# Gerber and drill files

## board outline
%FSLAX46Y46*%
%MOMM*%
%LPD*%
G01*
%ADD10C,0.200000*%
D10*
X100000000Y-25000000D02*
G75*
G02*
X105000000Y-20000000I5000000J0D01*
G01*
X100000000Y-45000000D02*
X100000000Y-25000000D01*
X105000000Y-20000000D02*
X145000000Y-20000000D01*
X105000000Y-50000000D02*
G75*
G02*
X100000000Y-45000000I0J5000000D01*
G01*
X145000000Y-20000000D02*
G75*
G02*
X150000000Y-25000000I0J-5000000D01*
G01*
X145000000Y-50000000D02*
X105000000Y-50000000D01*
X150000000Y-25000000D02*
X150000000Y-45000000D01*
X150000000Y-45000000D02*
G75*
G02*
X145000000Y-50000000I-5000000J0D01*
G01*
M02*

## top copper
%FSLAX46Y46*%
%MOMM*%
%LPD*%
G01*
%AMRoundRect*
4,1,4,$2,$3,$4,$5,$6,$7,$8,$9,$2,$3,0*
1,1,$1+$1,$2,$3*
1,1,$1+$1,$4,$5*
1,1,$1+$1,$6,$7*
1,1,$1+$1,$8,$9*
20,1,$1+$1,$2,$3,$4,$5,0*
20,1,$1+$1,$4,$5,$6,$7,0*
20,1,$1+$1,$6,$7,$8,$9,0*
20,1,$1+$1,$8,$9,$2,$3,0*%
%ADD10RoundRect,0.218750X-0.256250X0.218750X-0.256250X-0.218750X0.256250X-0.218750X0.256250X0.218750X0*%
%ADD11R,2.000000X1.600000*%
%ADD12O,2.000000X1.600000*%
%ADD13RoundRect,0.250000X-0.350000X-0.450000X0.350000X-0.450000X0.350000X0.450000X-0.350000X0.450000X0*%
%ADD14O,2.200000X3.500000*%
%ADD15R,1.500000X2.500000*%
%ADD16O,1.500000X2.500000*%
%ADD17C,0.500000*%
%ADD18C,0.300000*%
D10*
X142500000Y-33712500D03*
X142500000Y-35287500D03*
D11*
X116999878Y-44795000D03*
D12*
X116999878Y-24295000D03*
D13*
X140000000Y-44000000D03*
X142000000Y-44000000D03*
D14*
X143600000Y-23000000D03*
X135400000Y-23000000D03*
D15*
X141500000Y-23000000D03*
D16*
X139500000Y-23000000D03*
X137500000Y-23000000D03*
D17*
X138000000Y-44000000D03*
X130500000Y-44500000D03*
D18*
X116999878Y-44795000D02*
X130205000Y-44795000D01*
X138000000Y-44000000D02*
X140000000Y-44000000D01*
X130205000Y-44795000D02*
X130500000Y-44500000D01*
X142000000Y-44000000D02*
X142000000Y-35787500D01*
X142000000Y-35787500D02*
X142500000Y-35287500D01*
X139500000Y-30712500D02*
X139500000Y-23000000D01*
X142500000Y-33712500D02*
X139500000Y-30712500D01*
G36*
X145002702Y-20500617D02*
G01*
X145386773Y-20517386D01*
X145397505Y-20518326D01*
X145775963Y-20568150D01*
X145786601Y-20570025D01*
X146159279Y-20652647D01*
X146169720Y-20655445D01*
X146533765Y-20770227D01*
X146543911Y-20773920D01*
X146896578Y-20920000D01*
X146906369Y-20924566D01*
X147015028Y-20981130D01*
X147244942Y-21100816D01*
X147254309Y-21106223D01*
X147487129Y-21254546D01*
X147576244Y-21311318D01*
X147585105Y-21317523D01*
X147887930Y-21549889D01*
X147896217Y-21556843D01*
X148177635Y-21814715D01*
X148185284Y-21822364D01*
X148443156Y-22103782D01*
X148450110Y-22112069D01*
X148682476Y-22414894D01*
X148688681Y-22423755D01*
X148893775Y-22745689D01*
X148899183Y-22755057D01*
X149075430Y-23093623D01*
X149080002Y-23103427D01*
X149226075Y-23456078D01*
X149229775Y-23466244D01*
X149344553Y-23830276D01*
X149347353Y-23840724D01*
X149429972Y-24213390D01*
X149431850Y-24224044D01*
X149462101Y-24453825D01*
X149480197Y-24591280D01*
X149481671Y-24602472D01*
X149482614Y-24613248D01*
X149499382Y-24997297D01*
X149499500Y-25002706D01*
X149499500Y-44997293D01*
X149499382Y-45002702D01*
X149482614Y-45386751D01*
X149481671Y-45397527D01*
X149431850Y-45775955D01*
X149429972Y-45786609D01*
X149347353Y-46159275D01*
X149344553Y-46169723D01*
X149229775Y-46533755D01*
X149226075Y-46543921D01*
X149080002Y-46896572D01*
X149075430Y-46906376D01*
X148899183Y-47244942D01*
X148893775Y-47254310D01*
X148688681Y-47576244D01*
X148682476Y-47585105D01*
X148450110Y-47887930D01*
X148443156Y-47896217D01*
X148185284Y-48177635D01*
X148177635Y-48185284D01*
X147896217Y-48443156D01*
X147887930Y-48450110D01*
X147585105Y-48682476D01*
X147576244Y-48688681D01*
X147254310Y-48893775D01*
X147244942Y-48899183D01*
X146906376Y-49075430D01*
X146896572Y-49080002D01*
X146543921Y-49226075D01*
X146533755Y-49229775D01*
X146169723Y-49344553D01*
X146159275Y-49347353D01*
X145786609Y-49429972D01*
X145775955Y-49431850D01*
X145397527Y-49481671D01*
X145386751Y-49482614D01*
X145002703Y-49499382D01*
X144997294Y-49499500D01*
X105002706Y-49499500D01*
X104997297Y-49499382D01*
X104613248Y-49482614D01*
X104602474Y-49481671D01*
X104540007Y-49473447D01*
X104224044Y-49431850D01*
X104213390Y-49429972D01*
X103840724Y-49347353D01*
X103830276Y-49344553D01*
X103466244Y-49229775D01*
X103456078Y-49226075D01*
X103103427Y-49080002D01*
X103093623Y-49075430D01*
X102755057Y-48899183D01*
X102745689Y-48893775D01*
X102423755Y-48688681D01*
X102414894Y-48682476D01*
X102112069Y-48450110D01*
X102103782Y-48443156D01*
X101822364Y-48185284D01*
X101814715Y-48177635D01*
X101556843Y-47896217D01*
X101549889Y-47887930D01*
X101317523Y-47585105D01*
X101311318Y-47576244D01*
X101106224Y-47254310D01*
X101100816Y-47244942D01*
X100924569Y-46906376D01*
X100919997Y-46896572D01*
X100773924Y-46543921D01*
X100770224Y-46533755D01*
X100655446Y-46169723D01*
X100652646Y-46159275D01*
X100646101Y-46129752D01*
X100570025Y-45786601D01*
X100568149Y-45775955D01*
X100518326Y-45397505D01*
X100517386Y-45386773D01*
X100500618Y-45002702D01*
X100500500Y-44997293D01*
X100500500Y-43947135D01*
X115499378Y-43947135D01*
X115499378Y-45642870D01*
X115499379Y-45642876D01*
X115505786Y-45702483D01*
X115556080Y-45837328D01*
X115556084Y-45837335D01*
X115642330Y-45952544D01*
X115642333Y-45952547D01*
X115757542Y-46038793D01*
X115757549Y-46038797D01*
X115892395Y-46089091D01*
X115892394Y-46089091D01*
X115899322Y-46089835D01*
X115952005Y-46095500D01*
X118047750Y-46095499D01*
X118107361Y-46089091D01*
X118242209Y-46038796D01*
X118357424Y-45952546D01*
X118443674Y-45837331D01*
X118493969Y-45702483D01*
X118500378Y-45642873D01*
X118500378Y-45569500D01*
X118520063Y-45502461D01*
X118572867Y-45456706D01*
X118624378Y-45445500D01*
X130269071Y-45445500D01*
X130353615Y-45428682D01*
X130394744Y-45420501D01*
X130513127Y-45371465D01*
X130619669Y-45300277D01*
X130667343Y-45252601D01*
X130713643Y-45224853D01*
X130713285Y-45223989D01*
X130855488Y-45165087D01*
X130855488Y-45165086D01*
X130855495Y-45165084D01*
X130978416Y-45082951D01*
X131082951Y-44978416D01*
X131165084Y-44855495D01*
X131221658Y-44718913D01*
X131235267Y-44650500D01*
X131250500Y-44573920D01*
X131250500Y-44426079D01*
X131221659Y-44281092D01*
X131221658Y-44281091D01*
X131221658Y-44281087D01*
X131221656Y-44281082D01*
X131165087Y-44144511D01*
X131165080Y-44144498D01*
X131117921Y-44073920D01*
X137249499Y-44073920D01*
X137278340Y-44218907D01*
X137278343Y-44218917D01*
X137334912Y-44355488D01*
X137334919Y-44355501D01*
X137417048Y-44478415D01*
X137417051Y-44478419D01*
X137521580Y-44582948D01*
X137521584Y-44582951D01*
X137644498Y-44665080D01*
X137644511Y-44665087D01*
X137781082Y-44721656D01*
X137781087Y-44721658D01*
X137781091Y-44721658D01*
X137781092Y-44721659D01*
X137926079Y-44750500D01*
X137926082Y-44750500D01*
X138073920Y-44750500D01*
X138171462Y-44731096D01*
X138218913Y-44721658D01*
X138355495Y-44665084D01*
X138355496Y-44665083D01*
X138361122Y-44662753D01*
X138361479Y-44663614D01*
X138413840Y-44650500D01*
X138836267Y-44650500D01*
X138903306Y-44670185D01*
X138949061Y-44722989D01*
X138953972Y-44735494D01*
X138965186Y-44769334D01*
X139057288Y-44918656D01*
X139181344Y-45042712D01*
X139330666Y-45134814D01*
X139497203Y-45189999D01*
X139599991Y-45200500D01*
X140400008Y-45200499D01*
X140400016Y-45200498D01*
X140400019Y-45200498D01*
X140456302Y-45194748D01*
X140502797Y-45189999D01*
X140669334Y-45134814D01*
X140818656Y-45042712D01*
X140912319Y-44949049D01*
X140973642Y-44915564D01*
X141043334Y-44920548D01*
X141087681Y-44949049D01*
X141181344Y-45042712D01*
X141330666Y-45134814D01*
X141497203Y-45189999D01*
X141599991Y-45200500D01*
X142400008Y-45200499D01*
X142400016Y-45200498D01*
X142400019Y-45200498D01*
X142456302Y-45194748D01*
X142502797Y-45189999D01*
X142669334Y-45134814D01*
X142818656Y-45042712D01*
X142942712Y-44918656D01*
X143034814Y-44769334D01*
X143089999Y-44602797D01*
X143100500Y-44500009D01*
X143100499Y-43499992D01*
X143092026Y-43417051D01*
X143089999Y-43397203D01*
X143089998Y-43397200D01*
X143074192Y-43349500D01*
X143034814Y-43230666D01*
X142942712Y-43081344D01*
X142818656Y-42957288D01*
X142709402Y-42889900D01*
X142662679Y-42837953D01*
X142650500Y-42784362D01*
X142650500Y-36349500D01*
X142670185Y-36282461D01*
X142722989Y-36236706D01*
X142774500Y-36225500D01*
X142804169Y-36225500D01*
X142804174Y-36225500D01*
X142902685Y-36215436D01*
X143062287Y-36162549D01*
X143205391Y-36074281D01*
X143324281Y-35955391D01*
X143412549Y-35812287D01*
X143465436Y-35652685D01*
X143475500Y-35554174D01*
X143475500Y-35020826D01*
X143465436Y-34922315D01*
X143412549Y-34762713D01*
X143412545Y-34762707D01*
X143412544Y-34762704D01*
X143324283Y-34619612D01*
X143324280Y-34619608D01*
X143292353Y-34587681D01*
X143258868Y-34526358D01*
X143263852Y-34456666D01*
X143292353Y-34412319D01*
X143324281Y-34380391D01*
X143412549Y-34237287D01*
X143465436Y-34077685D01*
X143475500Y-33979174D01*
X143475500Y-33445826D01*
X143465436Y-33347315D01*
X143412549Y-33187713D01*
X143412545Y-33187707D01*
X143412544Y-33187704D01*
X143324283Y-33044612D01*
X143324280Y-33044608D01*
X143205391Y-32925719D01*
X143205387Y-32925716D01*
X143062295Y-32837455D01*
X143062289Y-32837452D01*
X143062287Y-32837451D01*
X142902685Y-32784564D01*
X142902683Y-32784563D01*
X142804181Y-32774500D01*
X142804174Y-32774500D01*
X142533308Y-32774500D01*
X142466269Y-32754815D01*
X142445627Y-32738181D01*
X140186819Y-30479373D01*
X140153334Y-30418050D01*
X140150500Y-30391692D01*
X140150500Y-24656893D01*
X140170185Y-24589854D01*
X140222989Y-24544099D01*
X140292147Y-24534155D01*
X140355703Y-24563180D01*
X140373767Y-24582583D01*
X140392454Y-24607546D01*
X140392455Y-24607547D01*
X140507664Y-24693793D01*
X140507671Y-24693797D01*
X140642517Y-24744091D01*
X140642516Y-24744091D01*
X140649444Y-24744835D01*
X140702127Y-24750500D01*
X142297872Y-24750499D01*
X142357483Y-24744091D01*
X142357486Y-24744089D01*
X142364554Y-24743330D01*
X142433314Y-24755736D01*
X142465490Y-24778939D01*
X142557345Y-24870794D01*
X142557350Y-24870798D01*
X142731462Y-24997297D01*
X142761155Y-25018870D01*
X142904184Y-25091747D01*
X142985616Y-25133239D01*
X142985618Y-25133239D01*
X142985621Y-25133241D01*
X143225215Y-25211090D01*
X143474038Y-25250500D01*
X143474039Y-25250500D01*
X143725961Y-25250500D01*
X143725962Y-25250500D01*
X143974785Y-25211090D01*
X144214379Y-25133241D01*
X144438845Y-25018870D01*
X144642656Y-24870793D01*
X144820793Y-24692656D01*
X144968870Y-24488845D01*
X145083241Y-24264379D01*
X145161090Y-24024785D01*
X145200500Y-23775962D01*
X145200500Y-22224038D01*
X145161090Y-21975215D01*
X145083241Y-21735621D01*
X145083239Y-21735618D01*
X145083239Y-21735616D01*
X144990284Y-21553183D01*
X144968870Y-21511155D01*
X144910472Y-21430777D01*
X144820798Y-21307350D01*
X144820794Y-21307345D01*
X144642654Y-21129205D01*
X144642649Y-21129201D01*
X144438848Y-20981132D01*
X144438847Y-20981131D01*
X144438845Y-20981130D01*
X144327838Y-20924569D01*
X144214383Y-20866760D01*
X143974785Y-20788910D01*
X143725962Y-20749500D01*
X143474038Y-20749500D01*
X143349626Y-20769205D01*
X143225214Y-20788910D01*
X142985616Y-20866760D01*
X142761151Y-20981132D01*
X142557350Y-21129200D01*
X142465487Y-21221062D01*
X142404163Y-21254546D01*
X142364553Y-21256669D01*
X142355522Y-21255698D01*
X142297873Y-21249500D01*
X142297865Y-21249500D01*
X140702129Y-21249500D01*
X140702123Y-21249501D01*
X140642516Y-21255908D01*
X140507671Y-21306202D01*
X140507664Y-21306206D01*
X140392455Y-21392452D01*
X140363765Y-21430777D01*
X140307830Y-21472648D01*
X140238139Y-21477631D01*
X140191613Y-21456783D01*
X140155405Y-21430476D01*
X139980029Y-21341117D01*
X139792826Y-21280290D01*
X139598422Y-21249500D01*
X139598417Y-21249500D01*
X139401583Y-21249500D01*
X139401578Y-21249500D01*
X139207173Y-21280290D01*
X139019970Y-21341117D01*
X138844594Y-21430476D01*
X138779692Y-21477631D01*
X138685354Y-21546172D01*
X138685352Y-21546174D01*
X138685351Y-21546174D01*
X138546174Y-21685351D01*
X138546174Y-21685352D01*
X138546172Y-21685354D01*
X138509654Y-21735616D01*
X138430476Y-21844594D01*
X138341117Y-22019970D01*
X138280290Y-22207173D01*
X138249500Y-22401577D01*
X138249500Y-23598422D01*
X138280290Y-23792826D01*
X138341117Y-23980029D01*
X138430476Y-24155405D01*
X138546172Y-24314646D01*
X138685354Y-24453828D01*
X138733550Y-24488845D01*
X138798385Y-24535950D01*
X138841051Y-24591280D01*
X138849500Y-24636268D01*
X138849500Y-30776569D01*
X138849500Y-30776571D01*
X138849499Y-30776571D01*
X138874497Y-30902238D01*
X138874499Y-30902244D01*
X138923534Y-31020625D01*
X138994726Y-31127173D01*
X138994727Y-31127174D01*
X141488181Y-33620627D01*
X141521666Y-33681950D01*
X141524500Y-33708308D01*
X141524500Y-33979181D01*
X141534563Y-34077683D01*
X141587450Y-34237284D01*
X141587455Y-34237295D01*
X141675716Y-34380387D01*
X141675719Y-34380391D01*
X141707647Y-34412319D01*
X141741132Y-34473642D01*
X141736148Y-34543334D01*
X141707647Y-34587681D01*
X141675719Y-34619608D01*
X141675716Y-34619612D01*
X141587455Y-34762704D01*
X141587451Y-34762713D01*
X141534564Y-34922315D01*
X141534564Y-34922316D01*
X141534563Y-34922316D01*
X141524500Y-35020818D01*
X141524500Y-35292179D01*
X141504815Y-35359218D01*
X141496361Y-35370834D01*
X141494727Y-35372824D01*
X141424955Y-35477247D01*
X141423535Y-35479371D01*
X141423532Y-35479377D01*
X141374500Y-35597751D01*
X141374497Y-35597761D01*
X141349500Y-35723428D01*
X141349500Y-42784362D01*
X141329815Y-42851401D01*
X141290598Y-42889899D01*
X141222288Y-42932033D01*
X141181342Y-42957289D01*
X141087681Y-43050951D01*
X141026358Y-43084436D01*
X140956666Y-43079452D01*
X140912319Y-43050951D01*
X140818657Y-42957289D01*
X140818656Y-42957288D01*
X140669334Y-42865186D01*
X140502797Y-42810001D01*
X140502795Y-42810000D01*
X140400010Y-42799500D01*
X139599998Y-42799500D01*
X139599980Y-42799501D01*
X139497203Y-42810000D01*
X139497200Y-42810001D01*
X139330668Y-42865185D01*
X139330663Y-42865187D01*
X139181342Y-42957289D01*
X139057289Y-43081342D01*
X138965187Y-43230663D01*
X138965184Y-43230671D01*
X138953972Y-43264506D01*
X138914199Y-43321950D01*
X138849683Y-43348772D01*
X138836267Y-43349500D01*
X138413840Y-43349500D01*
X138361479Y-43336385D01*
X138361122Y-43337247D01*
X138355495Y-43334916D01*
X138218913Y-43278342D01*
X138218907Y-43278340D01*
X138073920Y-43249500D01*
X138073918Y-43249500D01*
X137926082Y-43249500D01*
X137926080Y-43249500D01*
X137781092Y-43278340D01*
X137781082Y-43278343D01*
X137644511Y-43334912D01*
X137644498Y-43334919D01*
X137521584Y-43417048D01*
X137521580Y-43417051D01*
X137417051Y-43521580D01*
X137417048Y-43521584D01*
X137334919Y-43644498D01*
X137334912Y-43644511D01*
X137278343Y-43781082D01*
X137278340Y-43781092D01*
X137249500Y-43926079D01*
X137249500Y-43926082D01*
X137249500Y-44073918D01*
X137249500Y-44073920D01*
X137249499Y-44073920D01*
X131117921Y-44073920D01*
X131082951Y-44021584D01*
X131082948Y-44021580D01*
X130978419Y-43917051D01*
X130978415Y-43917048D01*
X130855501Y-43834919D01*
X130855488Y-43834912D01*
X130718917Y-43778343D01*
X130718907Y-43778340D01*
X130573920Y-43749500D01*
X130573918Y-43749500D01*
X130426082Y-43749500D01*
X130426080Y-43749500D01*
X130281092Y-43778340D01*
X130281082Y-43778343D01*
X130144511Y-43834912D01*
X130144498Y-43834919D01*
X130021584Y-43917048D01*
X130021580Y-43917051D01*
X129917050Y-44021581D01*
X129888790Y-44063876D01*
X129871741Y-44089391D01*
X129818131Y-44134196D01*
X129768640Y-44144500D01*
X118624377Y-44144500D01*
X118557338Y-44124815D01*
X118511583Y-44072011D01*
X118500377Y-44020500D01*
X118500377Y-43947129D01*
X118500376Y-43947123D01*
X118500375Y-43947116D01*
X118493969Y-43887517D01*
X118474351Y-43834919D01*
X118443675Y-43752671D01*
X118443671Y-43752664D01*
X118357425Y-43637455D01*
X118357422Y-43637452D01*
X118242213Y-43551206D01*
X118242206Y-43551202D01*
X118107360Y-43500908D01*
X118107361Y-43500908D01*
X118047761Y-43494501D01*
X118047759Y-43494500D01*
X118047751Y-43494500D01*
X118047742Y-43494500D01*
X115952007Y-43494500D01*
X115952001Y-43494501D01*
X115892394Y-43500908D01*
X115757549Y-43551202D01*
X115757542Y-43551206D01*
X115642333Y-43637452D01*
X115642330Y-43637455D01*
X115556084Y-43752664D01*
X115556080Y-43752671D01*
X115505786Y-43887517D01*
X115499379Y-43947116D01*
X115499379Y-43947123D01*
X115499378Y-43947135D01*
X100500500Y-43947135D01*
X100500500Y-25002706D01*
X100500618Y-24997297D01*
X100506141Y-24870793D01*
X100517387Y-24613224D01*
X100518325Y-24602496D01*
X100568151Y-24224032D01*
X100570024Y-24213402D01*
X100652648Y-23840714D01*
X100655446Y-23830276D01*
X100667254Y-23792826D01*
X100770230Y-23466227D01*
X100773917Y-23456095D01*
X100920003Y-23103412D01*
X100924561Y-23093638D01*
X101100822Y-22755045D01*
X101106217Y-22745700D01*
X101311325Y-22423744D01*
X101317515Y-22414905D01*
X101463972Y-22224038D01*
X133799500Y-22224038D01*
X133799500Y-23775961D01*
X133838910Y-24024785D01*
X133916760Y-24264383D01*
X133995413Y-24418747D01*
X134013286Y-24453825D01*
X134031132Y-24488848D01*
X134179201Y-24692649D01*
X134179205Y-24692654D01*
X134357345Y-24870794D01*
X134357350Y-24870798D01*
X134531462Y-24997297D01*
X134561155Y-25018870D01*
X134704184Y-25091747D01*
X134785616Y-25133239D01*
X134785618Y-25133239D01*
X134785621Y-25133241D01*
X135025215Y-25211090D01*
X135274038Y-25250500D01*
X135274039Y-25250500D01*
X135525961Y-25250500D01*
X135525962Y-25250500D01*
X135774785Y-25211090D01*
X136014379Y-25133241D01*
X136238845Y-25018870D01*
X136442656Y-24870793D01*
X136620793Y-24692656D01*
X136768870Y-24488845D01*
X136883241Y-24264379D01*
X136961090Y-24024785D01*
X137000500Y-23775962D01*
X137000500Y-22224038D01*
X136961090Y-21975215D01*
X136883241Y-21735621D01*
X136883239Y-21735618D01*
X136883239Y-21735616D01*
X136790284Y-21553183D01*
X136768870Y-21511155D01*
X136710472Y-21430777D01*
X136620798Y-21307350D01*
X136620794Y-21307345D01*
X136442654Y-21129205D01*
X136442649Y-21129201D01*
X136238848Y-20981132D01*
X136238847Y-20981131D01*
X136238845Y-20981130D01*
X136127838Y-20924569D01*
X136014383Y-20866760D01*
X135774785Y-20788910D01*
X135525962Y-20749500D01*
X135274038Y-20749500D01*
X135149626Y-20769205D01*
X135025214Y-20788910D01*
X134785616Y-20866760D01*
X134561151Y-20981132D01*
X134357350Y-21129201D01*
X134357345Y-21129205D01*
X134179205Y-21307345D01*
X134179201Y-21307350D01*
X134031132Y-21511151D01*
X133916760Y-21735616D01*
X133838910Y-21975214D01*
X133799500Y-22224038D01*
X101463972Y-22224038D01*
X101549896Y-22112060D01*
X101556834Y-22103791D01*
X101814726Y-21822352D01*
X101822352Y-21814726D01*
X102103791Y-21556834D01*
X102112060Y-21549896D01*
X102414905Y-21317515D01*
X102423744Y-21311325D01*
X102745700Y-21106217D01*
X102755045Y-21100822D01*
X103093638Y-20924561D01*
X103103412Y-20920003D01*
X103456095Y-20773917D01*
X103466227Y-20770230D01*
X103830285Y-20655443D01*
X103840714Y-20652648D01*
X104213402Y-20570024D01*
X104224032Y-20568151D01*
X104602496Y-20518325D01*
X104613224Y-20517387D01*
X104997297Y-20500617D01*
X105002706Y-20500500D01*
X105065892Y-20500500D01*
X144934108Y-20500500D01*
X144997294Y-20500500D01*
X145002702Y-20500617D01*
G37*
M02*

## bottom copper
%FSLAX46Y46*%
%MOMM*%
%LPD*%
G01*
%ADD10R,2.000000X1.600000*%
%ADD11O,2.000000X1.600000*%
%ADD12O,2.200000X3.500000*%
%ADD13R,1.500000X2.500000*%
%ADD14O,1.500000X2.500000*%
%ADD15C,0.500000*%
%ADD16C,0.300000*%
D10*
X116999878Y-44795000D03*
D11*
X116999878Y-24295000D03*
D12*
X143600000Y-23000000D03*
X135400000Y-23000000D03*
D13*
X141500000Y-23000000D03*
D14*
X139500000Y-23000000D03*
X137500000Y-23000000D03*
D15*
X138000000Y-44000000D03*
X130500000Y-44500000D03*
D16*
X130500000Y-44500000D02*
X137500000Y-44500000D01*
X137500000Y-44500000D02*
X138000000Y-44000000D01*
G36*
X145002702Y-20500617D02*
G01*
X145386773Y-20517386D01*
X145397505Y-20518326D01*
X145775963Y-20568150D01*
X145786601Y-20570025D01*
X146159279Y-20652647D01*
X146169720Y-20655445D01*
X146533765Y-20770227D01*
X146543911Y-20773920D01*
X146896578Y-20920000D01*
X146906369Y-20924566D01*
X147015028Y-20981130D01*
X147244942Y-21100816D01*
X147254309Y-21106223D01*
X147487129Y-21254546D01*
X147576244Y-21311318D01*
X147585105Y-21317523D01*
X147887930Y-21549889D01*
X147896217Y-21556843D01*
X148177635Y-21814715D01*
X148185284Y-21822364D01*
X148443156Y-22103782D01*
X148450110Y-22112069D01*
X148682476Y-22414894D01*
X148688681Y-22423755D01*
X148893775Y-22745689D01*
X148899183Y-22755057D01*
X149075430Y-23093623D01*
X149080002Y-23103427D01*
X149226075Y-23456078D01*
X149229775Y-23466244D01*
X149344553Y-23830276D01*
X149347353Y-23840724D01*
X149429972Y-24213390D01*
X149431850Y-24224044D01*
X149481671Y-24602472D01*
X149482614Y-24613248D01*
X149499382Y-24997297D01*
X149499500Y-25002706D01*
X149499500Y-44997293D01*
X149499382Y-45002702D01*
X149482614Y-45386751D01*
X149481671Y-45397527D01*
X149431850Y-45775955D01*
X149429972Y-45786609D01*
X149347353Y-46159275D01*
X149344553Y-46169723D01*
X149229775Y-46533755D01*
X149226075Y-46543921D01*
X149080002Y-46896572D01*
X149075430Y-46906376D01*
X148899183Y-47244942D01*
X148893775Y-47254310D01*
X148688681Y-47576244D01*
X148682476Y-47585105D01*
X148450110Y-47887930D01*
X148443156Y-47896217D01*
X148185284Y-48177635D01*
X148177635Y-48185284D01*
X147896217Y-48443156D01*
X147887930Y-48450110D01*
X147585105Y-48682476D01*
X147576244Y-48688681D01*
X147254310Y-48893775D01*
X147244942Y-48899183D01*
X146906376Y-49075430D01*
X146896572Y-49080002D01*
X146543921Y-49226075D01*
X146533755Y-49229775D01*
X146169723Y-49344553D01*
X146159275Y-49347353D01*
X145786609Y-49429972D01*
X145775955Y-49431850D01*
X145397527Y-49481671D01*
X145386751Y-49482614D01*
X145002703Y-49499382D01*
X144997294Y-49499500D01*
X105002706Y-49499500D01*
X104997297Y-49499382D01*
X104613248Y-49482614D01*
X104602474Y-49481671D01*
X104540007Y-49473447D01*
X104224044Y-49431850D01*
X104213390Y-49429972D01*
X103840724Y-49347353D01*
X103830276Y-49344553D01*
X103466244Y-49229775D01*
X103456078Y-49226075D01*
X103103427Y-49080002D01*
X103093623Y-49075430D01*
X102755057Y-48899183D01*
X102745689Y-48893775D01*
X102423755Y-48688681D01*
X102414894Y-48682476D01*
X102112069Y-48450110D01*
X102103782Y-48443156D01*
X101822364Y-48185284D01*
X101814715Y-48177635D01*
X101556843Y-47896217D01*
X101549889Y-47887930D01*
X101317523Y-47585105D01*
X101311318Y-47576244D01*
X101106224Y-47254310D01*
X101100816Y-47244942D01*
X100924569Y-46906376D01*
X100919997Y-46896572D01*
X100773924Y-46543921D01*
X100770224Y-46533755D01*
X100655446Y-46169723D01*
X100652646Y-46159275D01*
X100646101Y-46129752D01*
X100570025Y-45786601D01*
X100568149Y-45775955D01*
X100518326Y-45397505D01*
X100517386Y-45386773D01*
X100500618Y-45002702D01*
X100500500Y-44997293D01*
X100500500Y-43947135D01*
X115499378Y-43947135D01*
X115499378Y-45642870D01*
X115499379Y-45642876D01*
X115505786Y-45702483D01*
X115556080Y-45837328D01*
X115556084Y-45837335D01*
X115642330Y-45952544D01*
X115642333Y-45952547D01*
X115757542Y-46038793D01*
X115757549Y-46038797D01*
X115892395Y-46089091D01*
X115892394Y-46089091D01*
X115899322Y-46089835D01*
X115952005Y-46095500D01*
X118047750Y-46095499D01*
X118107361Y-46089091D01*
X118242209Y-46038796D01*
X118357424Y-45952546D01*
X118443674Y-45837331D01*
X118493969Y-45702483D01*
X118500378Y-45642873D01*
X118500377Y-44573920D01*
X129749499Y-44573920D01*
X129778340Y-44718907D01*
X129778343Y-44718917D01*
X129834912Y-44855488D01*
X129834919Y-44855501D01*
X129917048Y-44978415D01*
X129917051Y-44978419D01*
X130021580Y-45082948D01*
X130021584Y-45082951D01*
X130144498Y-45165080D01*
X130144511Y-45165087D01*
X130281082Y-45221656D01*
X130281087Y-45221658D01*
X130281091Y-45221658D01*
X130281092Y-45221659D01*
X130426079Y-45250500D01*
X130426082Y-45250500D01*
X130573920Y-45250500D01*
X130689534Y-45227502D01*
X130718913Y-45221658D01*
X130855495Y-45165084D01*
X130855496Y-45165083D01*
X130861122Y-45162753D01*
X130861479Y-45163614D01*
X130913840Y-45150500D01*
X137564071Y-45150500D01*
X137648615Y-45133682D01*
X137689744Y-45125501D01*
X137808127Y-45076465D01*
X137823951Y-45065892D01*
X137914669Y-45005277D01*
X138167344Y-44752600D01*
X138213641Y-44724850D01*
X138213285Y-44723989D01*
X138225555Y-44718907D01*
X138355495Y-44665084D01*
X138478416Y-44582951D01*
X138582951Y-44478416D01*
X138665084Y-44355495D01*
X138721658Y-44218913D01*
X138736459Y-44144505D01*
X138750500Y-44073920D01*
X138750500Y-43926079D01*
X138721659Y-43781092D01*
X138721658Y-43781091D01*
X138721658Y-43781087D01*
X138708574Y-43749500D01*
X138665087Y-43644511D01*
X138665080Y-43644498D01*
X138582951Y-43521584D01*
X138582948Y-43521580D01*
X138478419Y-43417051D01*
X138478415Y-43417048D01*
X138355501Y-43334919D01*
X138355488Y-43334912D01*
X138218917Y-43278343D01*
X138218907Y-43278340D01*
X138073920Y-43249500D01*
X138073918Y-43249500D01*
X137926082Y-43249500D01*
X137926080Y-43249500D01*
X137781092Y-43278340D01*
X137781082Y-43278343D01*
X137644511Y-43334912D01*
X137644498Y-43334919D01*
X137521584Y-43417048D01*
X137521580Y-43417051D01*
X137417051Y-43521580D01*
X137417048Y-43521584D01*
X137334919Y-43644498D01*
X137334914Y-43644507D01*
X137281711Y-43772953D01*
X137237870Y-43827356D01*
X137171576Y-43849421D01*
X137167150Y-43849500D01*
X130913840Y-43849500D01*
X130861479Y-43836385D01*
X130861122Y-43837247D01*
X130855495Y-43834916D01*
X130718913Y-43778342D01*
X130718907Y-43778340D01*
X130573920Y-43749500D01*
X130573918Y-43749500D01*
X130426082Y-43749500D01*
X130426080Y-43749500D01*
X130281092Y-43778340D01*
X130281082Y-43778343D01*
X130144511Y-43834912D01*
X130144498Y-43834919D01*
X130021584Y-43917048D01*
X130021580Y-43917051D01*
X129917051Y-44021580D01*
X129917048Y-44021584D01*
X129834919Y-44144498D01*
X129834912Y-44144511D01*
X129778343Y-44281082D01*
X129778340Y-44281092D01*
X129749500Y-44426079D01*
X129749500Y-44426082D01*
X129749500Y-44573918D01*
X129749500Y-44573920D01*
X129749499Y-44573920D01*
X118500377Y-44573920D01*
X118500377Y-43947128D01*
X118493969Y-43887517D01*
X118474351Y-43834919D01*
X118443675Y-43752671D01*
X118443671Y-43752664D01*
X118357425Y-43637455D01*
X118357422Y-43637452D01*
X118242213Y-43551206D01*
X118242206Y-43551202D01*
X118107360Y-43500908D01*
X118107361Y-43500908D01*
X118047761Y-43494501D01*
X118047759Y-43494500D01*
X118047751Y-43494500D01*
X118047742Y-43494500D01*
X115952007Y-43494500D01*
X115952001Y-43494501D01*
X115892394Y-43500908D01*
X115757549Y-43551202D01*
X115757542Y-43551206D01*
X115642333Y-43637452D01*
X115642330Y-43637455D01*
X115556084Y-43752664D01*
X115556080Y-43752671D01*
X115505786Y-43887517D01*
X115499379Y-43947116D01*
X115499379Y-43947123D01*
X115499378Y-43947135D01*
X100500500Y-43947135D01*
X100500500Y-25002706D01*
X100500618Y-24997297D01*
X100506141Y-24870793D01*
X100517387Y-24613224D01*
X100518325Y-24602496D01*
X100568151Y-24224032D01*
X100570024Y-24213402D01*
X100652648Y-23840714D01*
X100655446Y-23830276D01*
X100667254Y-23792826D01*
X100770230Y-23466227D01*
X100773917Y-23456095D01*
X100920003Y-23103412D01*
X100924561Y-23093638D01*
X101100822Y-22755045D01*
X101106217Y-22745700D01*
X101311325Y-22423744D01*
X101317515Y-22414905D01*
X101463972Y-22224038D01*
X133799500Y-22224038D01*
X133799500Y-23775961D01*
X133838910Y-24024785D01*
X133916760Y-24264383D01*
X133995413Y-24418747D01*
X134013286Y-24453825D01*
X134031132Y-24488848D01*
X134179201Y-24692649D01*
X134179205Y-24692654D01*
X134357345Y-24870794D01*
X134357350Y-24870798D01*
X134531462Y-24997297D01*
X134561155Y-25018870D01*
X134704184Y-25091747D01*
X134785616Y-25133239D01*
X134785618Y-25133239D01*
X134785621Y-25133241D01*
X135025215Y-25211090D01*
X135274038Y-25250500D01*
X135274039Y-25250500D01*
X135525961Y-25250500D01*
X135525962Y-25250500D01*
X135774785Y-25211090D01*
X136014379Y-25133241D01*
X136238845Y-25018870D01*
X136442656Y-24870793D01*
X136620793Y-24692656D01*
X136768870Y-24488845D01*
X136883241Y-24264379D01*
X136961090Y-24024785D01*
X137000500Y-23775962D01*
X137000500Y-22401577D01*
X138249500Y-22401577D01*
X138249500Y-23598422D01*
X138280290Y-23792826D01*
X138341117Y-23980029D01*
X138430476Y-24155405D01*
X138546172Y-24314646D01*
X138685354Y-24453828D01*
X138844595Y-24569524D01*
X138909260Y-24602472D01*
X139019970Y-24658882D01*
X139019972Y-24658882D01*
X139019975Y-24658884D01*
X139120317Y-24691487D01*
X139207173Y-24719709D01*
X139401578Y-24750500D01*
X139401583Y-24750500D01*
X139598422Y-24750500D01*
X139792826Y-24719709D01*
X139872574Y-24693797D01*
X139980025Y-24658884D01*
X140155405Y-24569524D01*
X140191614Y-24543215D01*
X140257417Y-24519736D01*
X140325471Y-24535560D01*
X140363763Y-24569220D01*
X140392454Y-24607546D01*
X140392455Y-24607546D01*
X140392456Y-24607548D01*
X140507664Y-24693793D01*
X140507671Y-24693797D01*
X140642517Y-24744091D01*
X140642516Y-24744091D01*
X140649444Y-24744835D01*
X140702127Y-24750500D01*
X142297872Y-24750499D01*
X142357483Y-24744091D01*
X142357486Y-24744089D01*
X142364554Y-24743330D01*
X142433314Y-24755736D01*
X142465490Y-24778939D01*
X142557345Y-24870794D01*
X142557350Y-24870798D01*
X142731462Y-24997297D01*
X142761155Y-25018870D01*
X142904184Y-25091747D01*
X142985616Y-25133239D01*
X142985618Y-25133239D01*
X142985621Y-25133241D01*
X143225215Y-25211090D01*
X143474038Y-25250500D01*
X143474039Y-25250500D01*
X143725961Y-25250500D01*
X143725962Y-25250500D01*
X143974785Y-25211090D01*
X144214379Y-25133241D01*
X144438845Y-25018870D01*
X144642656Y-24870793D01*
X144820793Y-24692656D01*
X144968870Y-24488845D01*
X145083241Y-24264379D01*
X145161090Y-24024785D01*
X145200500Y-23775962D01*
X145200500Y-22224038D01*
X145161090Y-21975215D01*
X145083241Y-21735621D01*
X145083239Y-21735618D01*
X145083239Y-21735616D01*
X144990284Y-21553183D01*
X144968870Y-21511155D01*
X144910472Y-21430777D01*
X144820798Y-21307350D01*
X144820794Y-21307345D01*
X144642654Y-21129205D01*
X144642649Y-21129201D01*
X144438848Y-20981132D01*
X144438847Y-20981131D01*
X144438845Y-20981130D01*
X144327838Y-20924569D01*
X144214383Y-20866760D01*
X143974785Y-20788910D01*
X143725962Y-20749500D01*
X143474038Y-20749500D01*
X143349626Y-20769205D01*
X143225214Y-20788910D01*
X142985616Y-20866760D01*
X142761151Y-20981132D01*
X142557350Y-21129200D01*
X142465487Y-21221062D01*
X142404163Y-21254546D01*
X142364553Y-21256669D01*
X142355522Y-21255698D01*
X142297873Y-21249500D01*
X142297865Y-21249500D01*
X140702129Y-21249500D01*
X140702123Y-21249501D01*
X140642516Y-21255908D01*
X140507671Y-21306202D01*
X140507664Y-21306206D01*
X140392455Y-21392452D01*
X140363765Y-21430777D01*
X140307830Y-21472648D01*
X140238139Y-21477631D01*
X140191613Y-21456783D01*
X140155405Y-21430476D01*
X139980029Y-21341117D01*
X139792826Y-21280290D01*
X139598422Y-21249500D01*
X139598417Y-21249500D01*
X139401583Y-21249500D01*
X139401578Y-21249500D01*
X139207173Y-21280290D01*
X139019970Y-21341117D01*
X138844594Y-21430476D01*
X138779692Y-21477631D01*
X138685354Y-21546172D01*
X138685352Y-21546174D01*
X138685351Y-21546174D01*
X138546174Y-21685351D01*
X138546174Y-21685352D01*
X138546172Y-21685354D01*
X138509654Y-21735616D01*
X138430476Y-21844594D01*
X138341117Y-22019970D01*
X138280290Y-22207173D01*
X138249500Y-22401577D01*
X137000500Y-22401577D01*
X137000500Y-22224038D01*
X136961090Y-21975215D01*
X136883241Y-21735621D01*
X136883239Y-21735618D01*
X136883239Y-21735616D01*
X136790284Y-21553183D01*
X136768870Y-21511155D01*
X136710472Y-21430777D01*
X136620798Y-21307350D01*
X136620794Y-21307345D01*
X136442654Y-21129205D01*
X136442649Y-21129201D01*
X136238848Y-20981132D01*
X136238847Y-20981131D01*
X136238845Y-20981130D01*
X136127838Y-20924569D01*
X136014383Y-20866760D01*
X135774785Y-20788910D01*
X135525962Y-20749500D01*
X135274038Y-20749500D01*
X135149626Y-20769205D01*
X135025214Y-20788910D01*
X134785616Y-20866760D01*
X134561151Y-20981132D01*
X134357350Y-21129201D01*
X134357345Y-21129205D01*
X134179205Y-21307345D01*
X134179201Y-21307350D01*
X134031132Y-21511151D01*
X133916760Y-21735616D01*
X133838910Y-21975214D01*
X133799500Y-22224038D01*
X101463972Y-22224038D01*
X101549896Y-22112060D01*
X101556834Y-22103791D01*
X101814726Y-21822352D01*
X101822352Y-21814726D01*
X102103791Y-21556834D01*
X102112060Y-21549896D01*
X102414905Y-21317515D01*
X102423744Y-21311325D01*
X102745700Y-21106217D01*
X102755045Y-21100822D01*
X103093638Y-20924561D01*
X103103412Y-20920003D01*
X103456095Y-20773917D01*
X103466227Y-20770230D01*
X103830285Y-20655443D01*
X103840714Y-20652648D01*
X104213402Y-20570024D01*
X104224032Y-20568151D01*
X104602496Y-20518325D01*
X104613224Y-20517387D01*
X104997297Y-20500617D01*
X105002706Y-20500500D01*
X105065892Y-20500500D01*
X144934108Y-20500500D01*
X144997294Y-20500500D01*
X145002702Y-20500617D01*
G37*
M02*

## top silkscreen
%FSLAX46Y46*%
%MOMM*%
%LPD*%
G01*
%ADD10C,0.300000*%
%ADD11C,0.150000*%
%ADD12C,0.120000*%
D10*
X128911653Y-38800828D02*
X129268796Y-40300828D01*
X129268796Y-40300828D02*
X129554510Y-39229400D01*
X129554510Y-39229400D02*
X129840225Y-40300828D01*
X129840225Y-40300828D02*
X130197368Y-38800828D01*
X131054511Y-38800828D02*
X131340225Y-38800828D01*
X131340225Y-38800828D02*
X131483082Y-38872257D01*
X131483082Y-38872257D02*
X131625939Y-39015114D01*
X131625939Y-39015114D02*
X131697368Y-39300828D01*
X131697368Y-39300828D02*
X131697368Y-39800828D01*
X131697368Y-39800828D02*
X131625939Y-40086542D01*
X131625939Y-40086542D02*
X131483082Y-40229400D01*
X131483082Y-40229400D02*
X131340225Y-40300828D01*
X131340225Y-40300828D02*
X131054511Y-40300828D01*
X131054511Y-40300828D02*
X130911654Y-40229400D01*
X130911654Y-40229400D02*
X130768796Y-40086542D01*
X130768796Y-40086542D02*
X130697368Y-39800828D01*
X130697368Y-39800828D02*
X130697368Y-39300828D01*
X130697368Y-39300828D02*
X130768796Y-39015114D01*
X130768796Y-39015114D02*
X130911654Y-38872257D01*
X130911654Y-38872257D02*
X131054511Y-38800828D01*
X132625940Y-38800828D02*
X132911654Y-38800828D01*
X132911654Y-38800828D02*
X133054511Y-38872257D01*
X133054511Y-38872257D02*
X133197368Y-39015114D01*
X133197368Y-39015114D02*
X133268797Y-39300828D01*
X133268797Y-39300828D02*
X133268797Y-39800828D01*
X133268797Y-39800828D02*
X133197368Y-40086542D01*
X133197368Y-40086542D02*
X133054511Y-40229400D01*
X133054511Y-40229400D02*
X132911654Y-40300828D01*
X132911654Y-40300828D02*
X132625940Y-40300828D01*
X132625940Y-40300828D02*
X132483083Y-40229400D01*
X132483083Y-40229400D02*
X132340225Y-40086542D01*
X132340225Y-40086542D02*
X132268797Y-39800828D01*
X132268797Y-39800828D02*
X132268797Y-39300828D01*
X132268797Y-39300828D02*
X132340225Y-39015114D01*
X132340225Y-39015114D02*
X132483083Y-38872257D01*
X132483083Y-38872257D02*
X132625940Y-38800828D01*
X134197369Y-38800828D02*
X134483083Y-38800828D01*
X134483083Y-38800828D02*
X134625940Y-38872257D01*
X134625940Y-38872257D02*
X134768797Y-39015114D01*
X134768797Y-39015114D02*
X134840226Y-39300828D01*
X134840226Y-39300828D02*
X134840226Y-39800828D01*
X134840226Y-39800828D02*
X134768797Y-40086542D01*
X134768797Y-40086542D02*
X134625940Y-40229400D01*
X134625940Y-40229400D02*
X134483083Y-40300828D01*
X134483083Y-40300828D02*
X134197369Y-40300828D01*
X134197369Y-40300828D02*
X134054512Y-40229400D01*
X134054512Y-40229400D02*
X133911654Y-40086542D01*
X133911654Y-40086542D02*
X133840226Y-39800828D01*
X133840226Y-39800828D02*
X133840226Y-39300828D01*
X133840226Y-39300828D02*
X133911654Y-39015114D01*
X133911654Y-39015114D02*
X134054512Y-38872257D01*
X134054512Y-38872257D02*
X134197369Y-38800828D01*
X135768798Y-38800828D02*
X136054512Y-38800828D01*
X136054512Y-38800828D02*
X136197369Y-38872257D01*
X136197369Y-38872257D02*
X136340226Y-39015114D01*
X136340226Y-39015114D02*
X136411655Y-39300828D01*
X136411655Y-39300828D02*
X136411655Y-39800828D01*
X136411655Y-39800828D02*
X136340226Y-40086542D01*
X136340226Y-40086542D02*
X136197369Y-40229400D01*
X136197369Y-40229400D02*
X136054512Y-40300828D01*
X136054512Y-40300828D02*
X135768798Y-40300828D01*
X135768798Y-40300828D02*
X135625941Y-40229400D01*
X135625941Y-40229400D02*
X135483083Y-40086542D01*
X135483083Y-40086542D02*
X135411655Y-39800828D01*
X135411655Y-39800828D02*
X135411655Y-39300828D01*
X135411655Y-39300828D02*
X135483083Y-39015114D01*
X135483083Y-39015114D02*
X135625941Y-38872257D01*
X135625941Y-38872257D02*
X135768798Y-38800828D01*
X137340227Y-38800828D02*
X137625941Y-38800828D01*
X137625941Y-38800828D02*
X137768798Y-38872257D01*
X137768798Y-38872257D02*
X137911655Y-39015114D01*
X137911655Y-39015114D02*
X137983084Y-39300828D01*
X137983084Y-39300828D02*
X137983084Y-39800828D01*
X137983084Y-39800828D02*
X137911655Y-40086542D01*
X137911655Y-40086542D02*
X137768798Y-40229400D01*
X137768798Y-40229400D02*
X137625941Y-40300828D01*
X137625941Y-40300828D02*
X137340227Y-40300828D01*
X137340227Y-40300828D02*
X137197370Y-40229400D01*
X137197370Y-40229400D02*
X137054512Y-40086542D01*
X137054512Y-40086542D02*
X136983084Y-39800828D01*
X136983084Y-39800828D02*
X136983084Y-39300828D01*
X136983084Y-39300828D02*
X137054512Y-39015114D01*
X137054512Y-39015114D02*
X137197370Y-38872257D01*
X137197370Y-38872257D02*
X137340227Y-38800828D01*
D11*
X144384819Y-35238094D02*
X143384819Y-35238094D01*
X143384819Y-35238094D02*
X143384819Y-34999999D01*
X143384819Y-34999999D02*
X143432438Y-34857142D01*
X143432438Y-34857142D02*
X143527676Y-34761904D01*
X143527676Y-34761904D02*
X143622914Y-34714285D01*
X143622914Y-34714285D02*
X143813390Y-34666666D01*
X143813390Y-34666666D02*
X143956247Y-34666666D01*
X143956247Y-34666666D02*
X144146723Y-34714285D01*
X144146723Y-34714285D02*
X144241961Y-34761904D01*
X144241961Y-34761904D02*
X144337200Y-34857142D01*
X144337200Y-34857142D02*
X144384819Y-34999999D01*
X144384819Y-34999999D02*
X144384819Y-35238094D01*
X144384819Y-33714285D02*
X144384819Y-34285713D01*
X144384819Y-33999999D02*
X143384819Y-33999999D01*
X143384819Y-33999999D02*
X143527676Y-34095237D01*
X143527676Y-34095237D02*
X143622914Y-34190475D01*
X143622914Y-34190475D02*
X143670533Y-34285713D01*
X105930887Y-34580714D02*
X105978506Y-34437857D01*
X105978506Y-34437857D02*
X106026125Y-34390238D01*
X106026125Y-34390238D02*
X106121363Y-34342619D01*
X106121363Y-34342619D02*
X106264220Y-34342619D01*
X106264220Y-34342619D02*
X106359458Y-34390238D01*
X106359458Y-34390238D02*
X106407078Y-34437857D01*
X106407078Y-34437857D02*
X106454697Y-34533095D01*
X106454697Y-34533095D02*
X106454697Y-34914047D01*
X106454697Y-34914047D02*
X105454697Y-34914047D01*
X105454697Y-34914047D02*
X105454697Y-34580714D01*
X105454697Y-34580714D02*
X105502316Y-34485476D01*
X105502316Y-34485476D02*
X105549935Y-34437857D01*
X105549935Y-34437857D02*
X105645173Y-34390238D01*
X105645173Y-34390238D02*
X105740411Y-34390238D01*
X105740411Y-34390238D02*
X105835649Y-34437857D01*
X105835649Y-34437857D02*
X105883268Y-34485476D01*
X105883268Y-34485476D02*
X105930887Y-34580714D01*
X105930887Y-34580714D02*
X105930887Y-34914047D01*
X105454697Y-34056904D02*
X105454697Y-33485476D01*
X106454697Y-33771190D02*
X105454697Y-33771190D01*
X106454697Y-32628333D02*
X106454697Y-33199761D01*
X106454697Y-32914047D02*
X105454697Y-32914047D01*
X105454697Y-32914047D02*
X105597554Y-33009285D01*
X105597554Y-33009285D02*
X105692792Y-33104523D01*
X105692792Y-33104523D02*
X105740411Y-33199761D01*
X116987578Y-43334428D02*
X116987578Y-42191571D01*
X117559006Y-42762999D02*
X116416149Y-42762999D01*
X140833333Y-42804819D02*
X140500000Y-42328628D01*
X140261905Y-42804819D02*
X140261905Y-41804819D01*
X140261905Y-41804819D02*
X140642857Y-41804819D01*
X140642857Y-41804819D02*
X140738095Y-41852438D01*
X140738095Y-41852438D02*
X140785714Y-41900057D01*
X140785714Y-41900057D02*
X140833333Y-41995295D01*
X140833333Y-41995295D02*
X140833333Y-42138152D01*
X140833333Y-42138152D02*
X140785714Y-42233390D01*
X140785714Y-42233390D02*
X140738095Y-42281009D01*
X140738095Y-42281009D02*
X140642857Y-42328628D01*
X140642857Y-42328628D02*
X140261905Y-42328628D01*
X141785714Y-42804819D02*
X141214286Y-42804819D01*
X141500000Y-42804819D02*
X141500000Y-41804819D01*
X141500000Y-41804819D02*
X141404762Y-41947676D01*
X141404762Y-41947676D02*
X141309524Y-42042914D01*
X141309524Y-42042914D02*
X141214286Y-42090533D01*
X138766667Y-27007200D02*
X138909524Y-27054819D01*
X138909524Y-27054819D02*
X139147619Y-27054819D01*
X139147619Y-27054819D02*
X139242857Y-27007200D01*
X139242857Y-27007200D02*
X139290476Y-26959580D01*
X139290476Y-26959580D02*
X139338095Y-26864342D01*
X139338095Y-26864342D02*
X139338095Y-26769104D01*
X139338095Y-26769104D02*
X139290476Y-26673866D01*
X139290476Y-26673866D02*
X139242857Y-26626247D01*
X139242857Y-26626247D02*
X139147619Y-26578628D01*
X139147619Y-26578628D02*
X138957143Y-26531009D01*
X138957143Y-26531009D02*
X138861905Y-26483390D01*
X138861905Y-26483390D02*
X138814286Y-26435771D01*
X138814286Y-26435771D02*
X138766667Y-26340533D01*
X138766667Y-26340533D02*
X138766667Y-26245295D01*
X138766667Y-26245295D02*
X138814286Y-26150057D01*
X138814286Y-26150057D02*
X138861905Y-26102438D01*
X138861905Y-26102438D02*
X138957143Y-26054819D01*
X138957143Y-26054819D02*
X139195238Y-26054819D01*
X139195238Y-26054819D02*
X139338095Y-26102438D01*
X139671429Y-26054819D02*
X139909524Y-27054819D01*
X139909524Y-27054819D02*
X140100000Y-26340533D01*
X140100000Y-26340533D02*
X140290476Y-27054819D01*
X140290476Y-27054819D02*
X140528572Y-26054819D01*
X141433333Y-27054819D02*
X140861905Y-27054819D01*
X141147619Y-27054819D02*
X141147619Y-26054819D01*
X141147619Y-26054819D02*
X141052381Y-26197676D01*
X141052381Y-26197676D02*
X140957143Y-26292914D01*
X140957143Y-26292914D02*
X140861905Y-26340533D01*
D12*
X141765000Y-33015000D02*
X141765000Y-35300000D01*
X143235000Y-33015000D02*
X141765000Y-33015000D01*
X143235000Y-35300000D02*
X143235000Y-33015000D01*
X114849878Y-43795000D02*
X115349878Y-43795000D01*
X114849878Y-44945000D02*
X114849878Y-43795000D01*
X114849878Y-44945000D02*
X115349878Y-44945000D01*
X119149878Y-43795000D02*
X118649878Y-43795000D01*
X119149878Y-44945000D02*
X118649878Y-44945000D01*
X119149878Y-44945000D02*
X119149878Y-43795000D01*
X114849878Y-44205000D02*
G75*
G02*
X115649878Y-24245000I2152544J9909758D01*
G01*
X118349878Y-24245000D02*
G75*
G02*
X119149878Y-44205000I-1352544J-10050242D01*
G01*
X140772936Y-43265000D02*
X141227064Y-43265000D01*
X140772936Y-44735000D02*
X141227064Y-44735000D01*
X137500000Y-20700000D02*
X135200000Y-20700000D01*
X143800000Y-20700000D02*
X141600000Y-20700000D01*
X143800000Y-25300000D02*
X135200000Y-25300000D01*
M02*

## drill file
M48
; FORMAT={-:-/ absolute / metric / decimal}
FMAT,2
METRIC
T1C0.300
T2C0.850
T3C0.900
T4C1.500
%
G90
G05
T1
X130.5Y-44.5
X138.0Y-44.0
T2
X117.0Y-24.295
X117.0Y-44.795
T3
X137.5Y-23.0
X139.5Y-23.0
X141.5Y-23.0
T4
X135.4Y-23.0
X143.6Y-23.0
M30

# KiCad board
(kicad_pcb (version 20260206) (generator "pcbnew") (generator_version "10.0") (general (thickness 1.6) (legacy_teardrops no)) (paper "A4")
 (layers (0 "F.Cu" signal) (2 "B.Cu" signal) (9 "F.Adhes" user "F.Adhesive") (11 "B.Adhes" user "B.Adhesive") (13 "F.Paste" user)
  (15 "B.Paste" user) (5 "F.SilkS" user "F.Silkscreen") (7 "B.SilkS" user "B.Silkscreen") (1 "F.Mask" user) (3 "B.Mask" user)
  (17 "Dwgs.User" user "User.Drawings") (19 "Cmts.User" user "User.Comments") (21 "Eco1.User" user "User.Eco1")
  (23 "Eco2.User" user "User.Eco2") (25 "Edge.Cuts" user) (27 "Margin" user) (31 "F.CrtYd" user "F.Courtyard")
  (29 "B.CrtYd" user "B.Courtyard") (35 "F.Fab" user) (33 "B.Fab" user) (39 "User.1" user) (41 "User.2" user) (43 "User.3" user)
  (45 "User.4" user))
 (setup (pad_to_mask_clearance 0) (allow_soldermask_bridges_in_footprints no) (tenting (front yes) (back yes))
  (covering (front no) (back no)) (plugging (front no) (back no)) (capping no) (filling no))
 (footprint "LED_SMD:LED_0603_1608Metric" (layer "F.Cu") (at 142.5 34.5 -90)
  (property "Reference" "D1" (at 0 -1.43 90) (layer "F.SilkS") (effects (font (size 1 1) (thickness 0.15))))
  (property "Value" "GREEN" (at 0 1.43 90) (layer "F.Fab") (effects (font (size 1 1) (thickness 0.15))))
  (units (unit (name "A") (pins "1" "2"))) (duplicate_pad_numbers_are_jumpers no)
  (fp_line (start -1.485 0.735) (end 0.8 0.735) (stroke (width 0.12) (type solid)) (layer "F.SilkS"))
  (fp_line (start -1.485 -0.735) (end -1.485 0.735) (stroke (width 0.12) (type solid)) (layer "F.SilkS"))
  (fp_line (start 0.8 -0.735) (end -1.485 -0.735) (stroke (width 0.12) (type solid)) (layer "F.SilkS"))
  (pad "1" smd roundrect (at -0.7875 0 270) (size 0.875 0.95) (layers "F.Cu" "F.Mask" "F.Paste") (roundrect_rratio 0.25) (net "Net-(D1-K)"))
  (pad "2" smd roundrect (at 0.7875 0 270) (size 0.875 0.95) (layers "F.Cu" "F.Mask" "F.Paste") (roundrect_rratio 0.25) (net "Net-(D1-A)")))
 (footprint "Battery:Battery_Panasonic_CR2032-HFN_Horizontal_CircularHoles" (layer "F.Cu") (at 116.999878 44.795 90)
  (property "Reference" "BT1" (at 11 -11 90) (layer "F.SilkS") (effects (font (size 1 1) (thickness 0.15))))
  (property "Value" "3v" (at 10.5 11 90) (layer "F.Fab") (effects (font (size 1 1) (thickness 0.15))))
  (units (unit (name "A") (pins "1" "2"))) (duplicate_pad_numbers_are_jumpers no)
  (fp_line (start 1 -2.15) (end 1 -1.65) (stroke (width 0.12) (type default)) (layer "F.SilkS"))
  (fp_line (start -0.15 -2.15) (end 1 -2.15) (stroke (width 0.12) (type default)) (layer "F.SilkS"))
  (fp_line (start -0.15 -2.15) (end -0.15 -1.65) (stroke (width 0.12) (type default)) (layer "F.SilkS"))
  (fp_line (start 1 2.15) (end 1 1.65) (stroke (width 0.12) (type default)) (layer "F.SilkS"))
  (fp_line (start -0.15 2.15) (end -0.15 1.65) (stroke (width 0.12) (type default)) (layer "F.SilkS"))
  (fp_line (start -0.15 2.15) (end 1 2.15) (stroke (width 0.12) (type default)) (layer "F.SilkS"))
  (fp_arc (start 0.59 -2.15) (mid 10.91 -10.13) (end 20.55 -1.35) (stroke (width 0.12) (type default)) (layer "F.SilkS"))
  (fp_arc (start 20.55 1.35) (mid 10.91 10.13) (end 0.59 2.15) (stroke (width 0.12) (type default)) (layer "F.SilkS"))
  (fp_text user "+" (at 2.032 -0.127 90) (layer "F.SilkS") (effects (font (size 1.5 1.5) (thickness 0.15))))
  (pad "1" thru_hole rect (at 0 0 90) (size 1.6 2) (drill 0.85) (layers "*.Cu" "*.Mask") (remove_unused_layers no) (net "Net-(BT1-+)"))
  (pad "2" thru_hole oval (at 20.5 0 90) (size 1.6 2) (drill 0.85) (layers "*.Cu" "*.Mask") (remove_unused_layers no) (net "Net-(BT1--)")))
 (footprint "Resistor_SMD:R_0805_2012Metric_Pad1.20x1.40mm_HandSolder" (layer "F.Cu") (at 141 44)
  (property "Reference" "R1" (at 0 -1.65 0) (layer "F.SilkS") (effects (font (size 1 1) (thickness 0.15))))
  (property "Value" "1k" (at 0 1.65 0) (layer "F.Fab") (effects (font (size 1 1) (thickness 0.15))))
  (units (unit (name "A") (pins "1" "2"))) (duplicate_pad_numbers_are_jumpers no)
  (fp_line (start -0.227064 -0.735) (end 0.227064 -0.735) (stroke (width 0.12) (type solid)) (layer "F.SilkS"))
  (fp_line (start -0.227064 0.735) (end 0.227064 0.735) (stroke (width 0.12) (type solid)) (layer "F.SilkS"))
  (pad "1" smd roundrect (at -1 0) (size 1.2 1.4) (layers "F.Cu" "F.Mask" "F.Paste") (roundrect_rratio 0.208333) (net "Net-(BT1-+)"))
  (pad "2" smd roundrect (at 1 0) (size 1.2 1.4) (layers "F.Cu" "F.Mask" "F.Paste") (roundrect_rratio 0.208333) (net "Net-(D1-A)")))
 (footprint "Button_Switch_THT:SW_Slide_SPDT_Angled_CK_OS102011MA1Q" (layer "F.Cu") (at 141.5 23 180)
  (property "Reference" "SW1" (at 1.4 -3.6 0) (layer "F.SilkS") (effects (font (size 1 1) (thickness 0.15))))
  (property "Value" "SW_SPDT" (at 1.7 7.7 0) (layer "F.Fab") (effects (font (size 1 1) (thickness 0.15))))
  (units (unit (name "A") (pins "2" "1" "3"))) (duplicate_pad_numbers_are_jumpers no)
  (fp_line (start 4 2.3) (end 6.3 2.3) (stroke (width 0.12) (type solid)) (layer "F.SilkS"))
  (fp_line (start -2.3 2.3) (end -0.1 2.3) (stroke (width 0.12) (type solid)) (layer "F.SilkS"))
  (fp_line (start -2.3 -2.3) (end 6.3 -2.3) (stroke (width 0.12) (type solid)) (layer "F.SilkS"))
  (pad "" thru_hole oval (at -2.1 0 180) (size 2.2 3.5) (drill 1.5) (layers "*.Cu" "*.Mask") (remove_unused_layers no))
  (pad "" thru_hole oval (at 6.1 0 180) (size 2.2 3.5) (drill 1.5) (layers "*.Cu" "*.Mask") (remove_unused_layers no))
  (pad "1" thru_hole rect (at 0 0 180) (size 1.5 2.5) (drill 0.9) (layers "*.Cu" "*.Mask") (remove_unused_layers no)
   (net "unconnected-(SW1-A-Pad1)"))
  (pad "2" thru_hole oval (at 2 0 180) (size 1.5 2.5) (drill 0.9) (layers "*.Cu" "*.Mask") (remove_unused_layers no) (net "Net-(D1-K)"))
  (pad "3" thru_hole oval (at 4 0 180) (size 1.5 2.5) (drill 0.9) (layers "*.Cu" "*.Mask") (remove_unused_layers no) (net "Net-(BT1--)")))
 (gr_arc (start 100 25) (mid 101.464466 21.464466) (end 105 20) (stroke (width 0.2) (type default)) (layer "Edge.Cuts"))
 (gr_line (start 100 45) (end 100 25) (stroke (width 0.2) (type default)) (layer "Edge.Cuts"))
 (gr_line (start 105 20) (end 145 20) (stroke (width 0.2) (type default)) (layer "Edge.Cuts"))
 (gr_arc (start 105 50) (mid 101.464466 48.535534) (end 100 45) (stroke (width 0.2) (type default)) (layer "Edge.Cuts"))
 (gr_arc (start 145 20) (mid 148.535534 21.464466) (end 150 25) (stroke (width 0.2) (type default)) (layer "Edge.Cuts"))
 (gr_line (start 145 50) (end 105 50) (stroke (width 0.2) (type default)) (layer "Edge.Cuts"))
 (gr_line (start 150 25) (end 150 45) (stroke (width 0.2) (type default)) (layer "Edge.Cuts"))
 (gr_arc (start 150 45) (mid 148.535534 48.535534) (end 145 50) (stroke (width 0.2) (type default)) (layer "Edge.Cuts"))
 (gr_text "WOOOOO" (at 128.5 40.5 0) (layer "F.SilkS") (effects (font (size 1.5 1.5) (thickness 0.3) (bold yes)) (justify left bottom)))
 (segment (start 116.999878 44.795) (end 130.205 44.795) (width 0.3) (layer "F.Cu") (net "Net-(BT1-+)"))
 (segment (start 138 44) (end 140 44) (width 0.3) (layer "F.Cu") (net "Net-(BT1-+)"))
 (segment (start 130.205 44.795) (end 130.5 44.5) (width 0.3) (layer "F.Cu") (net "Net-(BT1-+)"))
 (via (at 138 44) (size 0.5) (drill 0.3) (layers "F.Cu" "B.Cu") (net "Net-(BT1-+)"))
 (via (at 130.5 44.5) (size 0.5) (drill 0.3) (layers "F.Cu" "B.Cu") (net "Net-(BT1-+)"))
 (segment (start 130.5 44.5) (end 137.5 44.5) (width 0.3) (layer "B.Cu") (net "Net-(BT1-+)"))
 (segment (start 137.5 44.5) (end 138 44) (width 0.3) (layer "B.Cu") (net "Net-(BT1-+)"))
 (segment (start 142 44) (end 142 35.7875) (width 0.3) (layer "F.Cu") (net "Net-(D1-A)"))
 (segment (start 142 35.7875) (end 142.5 35.2875) (width 0.3) (layer "F.Cu") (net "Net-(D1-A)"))
 (segment (start 139.5 30.7125) (end 139.5 23) (width 0.3) (layer "F.Cu") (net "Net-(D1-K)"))
 (segment (start 142.5 33.7125) (end 139.5 30.7125) (width 0.3) (layer "F.Cu") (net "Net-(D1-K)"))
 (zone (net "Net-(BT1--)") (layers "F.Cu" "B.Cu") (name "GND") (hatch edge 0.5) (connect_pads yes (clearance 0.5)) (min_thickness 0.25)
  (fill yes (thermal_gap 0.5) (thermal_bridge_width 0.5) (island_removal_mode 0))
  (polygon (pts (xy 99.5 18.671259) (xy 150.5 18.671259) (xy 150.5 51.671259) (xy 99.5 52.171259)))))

